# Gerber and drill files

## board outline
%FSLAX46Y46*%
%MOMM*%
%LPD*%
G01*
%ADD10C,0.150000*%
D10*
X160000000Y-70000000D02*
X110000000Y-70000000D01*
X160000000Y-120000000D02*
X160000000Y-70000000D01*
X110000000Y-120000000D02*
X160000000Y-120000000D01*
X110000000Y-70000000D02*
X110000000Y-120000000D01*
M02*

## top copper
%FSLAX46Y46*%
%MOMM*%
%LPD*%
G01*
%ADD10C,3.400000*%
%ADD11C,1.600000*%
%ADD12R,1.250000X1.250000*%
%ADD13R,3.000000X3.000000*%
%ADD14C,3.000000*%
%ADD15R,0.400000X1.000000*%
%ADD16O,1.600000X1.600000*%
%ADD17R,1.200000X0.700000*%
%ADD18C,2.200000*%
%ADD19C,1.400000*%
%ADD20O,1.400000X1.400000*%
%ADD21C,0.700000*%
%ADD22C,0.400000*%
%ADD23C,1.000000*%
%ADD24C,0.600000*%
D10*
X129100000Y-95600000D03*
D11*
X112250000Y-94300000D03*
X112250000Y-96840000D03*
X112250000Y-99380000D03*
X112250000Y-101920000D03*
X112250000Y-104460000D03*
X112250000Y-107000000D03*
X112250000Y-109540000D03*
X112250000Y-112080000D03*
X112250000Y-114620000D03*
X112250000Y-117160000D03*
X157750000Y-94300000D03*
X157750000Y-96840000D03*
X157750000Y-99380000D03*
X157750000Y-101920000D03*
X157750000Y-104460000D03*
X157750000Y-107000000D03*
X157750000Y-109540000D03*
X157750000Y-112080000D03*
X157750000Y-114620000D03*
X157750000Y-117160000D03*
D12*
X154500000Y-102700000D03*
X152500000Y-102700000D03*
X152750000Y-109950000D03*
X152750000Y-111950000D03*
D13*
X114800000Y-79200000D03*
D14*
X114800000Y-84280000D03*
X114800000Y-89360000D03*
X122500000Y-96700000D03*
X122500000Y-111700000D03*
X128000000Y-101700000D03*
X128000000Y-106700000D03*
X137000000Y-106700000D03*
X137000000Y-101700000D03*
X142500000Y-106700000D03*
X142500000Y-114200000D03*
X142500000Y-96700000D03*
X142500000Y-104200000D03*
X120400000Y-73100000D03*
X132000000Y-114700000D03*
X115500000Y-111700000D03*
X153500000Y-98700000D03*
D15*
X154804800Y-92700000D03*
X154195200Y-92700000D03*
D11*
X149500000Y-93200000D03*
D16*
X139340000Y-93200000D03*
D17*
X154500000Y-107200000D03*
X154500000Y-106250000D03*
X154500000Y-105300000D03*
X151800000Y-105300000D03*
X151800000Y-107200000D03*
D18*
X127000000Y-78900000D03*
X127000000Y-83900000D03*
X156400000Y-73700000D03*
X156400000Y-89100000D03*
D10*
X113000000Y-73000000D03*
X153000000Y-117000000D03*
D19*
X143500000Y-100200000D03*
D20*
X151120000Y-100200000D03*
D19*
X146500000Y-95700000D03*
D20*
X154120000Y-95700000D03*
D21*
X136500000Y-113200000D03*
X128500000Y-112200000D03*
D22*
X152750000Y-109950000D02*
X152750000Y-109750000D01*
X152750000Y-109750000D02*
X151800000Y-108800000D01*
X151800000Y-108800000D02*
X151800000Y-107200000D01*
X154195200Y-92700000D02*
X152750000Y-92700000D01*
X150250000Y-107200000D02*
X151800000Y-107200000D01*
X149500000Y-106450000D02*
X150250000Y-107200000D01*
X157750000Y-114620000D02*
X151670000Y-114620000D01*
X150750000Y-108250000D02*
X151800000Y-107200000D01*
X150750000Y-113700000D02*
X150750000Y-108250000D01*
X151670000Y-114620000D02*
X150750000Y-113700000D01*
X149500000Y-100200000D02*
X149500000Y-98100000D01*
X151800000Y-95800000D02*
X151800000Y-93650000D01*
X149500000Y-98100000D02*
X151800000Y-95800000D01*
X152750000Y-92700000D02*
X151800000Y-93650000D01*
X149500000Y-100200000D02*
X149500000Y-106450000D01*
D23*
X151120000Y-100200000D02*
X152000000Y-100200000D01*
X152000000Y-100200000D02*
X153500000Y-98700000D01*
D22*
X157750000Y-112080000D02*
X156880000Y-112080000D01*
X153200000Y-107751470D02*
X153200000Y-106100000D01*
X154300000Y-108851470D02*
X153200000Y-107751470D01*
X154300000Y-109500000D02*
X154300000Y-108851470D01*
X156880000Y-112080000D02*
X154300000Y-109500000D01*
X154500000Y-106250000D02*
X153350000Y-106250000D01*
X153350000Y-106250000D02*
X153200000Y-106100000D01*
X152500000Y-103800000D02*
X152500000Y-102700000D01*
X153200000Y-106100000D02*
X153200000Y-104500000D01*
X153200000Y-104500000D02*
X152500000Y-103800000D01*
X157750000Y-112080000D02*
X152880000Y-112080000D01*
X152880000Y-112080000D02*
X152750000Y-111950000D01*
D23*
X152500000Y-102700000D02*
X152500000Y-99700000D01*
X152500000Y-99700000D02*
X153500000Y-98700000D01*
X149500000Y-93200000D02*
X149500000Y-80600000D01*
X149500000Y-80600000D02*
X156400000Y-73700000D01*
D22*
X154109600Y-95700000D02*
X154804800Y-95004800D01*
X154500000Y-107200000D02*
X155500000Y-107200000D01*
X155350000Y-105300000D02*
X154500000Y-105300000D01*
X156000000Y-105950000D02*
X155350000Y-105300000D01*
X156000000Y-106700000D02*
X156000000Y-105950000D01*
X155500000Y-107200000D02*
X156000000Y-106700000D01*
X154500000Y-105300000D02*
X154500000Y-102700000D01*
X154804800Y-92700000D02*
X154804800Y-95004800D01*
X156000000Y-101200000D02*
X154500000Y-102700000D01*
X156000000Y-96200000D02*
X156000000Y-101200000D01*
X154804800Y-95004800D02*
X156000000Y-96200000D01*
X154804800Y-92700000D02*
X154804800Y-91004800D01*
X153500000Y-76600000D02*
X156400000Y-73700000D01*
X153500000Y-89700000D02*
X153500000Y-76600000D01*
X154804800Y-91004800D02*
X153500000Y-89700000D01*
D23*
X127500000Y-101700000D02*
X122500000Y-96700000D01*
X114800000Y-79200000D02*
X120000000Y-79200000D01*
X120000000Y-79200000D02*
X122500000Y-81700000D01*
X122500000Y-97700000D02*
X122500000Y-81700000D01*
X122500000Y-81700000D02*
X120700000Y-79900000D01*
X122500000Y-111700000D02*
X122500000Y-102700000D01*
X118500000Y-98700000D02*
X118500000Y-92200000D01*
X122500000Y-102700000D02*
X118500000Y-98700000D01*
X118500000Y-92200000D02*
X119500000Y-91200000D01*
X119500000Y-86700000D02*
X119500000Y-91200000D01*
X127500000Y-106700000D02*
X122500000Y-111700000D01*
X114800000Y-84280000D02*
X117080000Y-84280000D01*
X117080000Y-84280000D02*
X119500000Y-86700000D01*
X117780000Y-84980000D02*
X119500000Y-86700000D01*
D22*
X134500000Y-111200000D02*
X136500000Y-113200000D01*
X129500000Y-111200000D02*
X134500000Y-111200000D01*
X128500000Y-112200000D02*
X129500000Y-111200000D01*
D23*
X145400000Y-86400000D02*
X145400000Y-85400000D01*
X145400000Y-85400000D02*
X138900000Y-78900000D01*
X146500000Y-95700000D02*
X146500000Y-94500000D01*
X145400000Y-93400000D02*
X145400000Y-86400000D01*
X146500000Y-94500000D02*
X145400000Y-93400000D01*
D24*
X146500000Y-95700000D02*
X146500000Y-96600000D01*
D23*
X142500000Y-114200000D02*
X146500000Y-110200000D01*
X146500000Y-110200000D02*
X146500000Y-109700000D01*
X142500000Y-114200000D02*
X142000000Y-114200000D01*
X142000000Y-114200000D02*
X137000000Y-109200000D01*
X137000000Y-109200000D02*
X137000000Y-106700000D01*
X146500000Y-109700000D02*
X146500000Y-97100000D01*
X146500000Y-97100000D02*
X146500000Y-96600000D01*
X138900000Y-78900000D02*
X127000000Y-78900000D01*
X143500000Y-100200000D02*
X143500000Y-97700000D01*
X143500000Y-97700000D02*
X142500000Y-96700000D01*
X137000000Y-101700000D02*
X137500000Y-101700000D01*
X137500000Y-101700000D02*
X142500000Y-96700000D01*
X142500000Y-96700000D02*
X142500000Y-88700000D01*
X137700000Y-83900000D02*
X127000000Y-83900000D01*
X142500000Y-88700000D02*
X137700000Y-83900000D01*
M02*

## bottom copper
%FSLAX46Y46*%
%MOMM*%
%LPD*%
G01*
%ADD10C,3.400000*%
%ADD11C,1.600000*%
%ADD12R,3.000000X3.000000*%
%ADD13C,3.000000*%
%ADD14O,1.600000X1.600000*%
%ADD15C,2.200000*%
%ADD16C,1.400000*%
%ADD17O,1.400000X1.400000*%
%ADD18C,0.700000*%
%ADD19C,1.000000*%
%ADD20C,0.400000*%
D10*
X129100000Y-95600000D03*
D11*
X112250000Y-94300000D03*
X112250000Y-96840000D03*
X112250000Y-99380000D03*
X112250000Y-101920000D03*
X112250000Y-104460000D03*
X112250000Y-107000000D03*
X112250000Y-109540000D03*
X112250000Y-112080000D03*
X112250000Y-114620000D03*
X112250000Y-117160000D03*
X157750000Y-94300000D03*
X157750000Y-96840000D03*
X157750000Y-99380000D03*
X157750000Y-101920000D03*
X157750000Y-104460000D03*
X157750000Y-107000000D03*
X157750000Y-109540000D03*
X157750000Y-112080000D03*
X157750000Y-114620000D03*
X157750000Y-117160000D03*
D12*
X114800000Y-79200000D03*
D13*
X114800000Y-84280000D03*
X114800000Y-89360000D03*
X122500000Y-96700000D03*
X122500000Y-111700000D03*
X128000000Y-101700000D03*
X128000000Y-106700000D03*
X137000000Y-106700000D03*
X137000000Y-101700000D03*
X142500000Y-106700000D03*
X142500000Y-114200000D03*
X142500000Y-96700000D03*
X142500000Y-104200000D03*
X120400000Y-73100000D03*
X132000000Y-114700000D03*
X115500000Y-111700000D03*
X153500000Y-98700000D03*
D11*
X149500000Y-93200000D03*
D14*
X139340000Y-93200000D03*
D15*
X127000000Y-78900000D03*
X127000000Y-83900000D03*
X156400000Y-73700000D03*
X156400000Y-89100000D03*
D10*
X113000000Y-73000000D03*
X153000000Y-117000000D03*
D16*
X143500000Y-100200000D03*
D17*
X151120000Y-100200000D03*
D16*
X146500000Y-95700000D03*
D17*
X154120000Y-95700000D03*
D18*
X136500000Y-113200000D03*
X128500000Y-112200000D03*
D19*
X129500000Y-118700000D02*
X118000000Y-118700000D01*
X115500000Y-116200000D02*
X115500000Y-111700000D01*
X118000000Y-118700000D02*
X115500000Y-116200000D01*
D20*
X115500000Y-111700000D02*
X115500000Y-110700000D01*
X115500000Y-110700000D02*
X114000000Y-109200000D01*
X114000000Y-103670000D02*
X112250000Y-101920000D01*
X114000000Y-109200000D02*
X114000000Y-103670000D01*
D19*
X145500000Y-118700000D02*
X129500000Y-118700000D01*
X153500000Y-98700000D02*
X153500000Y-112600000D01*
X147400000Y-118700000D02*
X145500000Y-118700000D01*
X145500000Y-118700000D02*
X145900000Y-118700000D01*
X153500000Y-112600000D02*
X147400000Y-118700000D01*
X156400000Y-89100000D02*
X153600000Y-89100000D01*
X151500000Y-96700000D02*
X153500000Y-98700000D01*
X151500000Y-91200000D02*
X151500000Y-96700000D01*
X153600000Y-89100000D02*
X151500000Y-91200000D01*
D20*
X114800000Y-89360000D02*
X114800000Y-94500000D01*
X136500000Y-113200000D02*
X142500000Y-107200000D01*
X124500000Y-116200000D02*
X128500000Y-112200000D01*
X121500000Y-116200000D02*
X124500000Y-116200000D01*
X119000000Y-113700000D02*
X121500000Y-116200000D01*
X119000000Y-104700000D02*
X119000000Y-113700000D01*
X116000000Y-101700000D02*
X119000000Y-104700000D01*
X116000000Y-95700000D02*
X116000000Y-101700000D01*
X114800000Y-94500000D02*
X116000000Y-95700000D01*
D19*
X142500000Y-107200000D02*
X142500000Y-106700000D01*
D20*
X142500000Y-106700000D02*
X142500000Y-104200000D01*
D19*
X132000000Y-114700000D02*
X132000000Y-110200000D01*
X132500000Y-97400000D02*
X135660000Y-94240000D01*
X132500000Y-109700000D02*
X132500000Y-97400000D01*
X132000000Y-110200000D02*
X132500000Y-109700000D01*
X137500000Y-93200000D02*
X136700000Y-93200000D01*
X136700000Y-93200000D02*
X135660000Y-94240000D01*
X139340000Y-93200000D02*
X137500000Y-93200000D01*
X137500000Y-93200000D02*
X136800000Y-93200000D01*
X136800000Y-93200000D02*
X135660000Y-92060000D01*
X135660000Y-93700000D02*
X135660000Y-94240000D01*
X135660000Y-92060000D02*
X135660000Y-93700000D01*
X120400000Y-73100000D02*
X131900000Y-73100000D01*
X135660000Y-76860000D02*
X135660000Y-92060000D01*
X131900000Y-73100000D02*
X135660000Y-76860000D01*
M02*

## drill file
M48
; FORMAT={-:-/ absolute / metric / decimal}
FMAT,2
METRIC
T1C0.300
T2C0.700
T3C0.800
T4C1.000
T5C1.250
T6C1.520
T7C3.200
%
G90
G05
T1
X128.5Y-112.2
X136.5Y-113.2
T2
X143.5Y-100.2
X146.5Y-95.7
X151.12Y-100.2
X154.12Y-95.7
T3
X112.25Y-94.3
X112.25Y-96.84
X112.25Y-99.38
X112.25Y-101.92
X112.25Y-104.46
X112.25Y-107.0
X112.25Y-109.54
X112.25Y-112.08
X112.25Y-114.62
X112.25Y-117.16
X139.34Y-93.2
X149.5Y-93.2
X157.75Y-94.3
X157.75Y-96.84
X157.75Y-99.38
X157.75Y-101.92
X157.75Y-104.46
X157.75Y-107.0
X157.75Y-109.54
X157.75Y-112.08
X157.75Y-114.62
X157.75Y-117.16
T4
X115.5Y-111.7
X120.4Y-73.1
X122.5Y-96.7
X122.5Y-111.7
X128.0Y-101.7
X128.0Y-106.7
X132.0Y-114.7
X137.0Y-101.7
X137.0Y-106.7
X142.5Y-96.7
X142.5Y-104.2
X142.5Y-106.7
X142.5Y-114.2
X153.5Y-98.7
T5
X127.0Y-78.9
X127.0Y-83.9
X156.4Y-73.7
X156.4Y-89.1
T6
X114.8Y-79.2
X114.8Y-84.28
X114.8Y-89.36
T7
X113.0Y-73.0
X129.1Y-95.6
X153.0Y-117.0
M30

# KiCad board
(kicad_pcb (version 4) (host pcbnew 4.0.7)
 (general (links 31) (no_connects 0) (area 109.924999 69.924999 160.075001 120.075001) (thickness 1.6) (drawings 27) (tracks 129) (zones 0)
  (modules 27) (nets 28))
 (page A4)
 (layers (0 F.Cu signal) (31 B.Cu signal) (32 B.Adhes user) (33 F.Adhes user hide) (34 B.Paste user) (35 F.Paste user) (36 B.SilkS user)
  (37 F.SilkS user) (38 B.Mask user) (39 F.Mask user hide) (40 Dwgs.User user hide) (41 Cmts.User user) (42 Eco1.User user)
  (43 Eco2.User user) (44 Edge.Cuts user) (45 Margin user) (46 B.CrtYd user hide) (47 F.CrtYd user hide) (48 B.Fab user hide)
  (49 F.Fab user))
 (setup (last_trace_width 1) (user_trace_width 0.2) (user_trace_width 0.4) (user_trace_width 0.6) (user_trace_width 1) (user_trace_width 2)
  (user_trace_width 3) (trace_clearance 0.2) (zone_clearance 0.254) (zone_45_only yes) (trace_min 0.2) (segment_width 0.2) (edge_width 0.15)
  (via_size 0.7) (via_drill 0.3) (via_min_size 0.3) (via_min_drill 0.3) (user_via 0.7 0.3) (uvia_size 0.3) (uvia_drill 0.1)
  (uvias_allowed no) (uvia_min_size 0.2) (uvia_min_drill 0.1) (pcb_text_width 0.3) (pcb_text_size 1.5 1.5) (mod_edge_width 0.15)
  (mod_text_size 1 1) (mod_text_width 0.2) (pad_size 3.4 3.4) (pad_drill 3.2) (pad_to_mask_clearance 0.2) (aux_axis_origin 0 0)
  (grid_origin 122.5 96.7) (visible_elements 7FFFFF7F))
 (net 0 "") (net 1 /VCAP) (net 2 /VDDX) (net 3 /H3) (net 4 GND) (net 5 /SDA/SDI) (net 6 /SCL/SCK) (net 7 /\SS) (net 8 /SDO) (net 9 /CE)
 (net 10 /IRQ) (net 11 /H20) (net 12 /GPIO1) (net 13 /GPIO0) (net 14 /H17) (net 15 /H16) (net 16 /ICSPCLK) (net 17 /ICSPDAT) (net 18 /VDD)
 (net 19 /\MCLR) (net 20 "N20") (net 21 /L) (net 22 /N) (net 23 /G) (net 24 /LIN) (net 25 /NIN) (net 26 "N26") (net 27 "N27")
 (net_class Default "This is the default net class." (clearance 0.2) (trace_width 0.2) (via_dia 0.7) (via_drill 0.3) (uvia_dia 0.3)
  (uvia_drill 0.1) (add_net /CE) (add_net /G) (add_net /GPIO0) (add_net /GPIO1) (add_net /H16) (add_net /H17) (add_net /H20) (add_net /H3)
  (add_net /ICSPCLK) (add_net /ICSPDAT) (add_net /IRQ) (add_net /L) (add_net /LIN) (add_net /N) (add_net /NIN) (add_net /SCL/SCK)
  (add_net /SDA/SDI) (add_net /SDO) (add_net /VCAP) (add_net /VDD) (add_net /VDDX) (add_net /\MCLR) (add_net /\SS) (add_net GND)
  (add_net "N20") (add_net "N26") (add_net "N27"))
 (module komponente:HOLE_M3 (layer F.Cu) (at 129.1 95.6)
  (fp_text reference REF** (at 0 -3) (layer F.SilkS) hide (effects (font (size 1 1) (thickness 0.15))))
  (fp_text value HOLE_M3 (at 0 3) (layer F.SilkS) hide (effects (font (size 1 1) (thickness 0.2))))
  (pad 1 thru_hole circle (at 0 0) (size 3.4 3.4) (drill 3.2) (layers *.Cu *.Mask F.SilkS)))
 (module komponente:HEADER (layer F.Cu) (at 135 107)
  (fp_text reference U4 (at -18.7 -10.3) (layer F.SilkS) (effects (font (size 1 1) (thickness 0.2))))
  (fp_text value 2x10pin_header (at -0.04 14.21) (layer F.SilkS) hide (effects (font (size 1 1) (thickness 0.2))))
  (pad 1 thru_hole circle (at -22.75 -12.7) (size 1.6 1.6) (drill 0.8) (layers *.Cu *.Mask F.SilkS) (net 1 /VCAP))
  (pad 2 thru_hole circle (at -22.75 -10.16) (size 1.6 1.6) (drill 0.8) (layers *.Cu *.Mask F.SilkS) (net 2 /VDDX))
  (pad 3 thru_hole circle (at -22.75 -7.62) (size 1.6 1.6) (drill 0.8) (layers *.Cu *.Mask F.SilkS) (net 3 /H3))
  (pad 4 thru_hole circle (at -22.75 -5.08) (size 1.6 1.6) (drill 0.8) (layers *.Cu *.Mask F.SilkS) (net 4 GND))
  (pad 5 thru_hole circle (at -22.75 -2.54) (size 1.6 1.6) (drill 0.8) (layers *.Cu *.Mask F.SilkS) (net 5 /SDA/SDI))
  (pad 6 thru_hole circle (at -22.75 0) (size 1.6 1.6) (drill 0.8) (layers *.Cu *.Mask F.SilkS) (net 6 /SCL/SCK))
  (pad 7 thru_hole circle (at -22.75 2.54) (size 1.6 1.6) (drill 0.8) (layers *.Cu *.Mask F.SilkS) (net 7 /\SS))
  (pad 8 thru_hole circle (at -22.75 5.08) (size 1.6 1.6) (drill 0.8) (layers *.Cu *.Mask F.SilkS) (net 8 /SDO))
  (pad 9 thru_hole circle (at -22.75 7.62) (size 1.6 1.6) (drill 0.8) (layers *.Cu *.Mask F.SilkS) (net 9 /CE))
  (pad 10 thru_hole circle (at -22.75 10.16) (size 1.6 1.6) (drill 0.8) (layers *.Cu *.Mask F.SilkS) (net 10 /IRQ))
  (pad 20 thru_hole circle (at 22.75 -12.7) (size 1.6 1.6) (drill 0.8) (layers *.Cu *.Mask F.SilkS) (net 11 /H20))
  (pad 19 thru_hole circle (at 22.75 -10.16) (size 1.6 1.6) (drill 0.8) (layers *.Cu *.Mask F.SilkS) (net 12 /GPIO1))
  (pad 18 thru_hole circle (at 22.75 -7.62) (size 1.6 1.6) (drill 0.8) (layers *.Cu *.Mask F.SilkS) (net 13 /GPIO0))
  (pad 17 thru_hole circle (at 22.75 -5.08) (size 1.6 1.6) (drill 0.8) (layers *.Cu *.Mask F.SilkS) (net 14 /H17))
  (pad 16 thru_hole circle (at 22.75 -2.54) (size 1.6 1.6) (drill 0.8) (layers *.Cu *.Mask F.SilkS) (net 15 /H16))
  (pad 15 thru_hole circle (at 22.75 0) (size 1.6 1.6) (drill 0.8) (layers *.Cu *.Mask F.SilkS) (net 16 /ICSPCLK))
  (pad 14 thru_hole circle (at 22.75 2.54) (size 1.6 1.6) (drill 0.8) (layers *.Cu *.Mask F.SilkS) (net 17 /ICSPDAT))
  (pad 13 thru_hole circle (at 22.75 5.08) (size 1.6 1.6) (drill 0.8) (layers *.Cu *.Mask F.SilkS) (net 4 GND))
  (pad 12 thru_hole circle (at 22.75 7.62) (size 1.6 1.6) (drill 0.8) (layers *.Cu *.Mask F.SilkS) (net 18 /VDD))
  (pad 11 thru_hole circle (at 22.75 10.16) (size 1.6 1.6) (drill 0.8) (layers *.Cu *.Mask F.SilkS) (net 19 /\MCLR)))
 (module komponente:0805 (layer F.Cu) (at 153.5 102.7 180)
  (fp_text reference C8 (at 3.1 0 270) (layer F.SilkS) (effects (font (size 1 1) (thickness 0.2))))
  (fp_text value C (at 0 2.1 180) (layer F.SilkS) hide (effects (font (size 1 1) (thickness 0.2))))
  (pad 1 smd rect (at -1 0 180) (size 1.25 1.25) (layers F.Cu F.Paste F.Mask) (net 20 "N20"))
  (pad 2 smd rect (at 1 0 180) (size 1.25 1.25) (layers F.Cu F.Paste F.Mask) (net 4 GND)))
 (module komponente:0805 (layer F.Cu) (at 152.75 110.95 270)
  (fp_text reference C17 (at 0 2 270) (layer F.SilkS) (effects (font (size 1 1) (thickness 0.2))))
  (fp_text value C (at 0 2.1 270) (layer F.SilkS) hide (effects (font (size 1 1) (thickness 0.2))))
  (pad 1 smd rect (at -1 0 270) (size 1.25 1.25) (layers F.Cu F.Paste F.Mask) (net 18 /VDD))
  (pad 2 smd rect (at 1 0 270) (size 1.25 1.25) (layers F.Cu F.Paste F.Mask) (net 4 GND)))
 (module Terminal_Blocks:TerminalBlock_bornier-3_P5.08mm (layer F.Cu) (at 114.8 79.2 270)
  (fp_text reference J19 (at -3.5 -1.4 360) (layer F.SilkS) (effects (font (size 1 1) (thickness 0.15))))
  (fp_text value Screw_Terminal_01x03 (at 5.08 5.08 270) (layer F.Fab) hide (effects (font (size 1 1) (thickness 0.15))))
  (pad 1 thru_hole rect (at 0 0 270) (size 3 3) (drill 1.52) (layers *.Cu *.Mask) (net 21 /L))
  (pad 2 thru_hole circle (at 5.08 0 270) (size 3 3) (drill 1.52) (layers *.Cu *.Mask) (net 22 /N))
  (pad 3 thru_hole circle (at 10.16 0 270) (size 3 3) (drill 1.52) (layers *.Cu *.Mask) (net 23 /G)))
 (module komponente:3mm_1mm (layer F.Cu) (at 122.5 96.7)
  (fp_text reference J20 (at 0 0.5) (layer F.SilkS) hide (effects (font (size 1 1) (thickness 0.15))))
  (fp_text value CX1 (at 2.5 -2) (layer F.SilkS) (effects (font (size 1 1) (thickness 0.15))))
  (pad 1 thru_hole circle (at 0 0) (size 3 3) (drill 1) (layers *.Cu *.Mask) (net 21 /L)))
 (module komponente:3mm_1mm (layer F.Cu) (at 122.5 111.7)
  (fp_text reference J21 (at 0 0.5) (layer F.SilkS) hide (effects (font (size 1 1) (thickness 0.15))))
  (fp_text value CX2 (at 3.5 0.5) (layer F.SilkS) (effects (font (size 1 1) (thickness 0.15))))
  (pad 1 thru_hole circle (at 0 0) (size 3 3) (drill 1) (layers *.Cu *.Mask) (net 22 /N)))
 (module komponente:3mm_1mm (layer F.Cu) (at 128 101.7)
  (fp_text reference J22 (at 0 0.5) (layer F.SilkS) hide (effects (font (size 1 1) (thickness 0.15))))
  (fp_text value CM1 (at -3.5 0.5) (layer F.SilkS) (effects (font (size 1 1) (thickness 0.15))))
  (pad 1 thru_hole circle (at 0 0) (size 3 3) (drill 1) (layers *.Cu *.Mask) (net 21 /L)))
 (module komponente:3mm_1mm (layer F.Cu) (at 128 106.7)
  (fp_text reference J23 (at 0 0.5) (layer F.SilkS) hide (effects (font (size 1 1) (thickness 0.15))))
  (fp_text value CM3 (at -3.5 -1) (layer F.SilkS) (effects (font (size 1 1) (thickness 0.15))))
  (pad 1 thru_hole circle (at 0 0) (size 3 3) (drill 1) (layers *.Cu *.Mask) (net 22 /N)))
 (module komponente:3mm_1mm (layer F.Cu) (at 137 106.7)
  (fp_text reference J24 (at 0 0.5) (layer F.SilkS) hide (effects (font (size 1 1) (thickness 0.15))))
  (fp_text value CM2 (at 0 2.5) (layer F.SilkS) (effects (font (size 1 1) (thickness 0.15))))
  (pad 1 thru_hole circle (at 0 0) (size 3 3) (drill 1) (layers *.Cu *.Mask) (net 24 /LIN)))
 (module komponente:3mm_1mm (layer F.Cu) (at 137 101.7)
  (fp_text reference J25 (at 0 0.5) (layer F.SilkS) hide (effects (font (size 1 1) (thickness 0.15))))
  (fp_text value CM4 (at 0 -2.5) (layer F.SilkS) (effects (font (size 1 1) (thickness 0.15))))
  (pad 1 thru_hole circle (at 0 0) (size 3 3) (drill 1) (layers *.Cu *.Mask) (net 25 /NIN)))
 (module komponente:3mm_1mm (layer F.Cu) (at 142.5 106.7)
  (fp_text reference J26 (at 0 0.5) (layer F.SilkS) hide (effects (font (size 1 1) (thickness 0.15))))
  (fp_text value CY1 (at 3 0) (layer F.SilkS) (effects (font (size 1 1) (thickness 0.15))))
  (pad 1 thru_hole circle (at 0 0) (size 3 3) (drill 1) (layers *.Cu *.Mask) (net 23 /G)))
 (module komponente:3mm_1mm (layer F.Cu) (at 142.5 114.2)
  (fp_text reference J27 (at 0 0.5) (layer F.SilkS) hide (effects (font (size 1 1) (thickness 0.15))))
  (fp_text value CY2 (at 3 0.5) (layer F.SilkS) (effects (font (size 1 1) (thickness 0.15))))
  (pad 1 thru_hole circle (at 0 0) (size 3 3) (drill 1) (layers *.Cu *.Mask) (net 24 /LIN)))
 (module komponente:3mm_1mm (layer F.Cu) (at 142.5 96.7)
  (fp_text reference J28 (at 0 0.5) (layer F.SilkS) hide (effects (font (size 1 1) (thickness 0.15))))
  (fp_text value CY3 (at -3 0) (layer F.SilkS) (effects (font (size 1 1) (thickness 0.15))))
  (pad 1 thru_hole circle (at 0 0) (size 3 3) (drill 1) (layers *.Cu *.Mask) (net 25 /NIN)))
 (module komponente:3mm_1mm (layer F.Cu) (at 142.5 104.2)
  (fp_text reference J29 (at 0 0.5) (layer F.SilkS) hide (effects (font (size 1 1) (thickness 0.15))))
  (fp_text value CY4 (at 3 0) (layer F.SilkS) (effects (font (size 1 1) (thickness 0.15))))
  (pad 1 thru_hole circle (at 0 0) (size 3 3) (drill 1) (layers *.Cu *.Mask) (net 23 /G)))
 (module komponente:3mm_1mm (layer F.Cu) (at 120.4 73.1)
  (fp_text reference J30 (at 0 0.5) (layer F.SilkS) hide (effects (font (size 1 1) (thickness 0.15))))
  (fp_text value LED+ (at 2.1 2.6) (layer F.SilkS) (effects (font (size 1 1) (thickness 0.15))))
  (pad 1 thru_hole circle (at 0 0) (size 3 3) (drill 1) (layers *.Cu *.Mask) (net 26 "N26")))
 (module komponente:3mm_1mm (layer F.Cu) (at 132 114.7)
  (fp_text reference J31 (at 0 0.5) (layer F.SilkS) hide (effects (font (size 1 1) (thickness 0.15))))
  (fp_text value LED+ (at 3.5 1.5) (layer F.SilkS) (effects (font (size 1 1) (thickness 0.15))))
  (pad 1 thru_hole circle (at 0 0) (size 3 3) (drill 1) (layers *.Cu *.Mask) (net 26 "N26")))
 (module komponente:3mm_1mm (layer F.Cu) (at 115.5 111.7)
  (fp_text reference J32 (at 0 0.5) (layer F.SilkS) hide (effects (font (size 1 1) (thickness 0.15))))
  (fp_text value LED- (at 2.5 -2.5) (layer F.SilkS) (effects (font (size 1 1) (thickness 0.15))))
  (pad 1 thru_hole circle (at 0 0) (size 3 3) (drill 1) (layers *.Cu *.Mask) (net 4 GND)))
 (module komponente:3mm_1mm (layer F.Cu) (at 153.5 98.7)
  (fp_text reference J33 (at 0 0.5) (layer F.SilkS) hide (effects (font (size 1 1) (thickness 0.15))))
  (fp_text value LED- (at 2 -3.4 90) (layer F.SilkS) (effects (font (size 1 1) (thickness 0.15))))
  (pad 1 thru_hole circle (at 0 0) (size 3 3) (drill 1) (layers *.Cu *.Mask) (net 4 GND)))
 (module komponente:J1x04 (layer F.Cu) (at 154.5 92.7 180)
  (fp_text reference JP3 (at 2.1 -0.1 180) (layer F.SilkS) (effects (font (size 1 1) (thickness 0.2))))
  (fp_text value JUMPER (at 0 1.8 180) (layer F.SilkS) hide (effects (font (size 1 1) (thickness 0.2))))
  (pad 1 smd rect (at -0.3048 0 180) (size 0.4 1) (layers F.Cu F.Paste F.Mask) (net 20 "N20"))
  (pad 2 smd rect (at 0.3048 0 180) (size 0.4 1) (layers F.Cu F.Paste F.Mask) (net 18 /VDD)))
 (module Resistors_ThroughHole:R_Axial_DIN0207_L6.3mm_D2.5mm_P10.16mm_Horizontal (layer F.Cu) (at 149.5 93.2 180)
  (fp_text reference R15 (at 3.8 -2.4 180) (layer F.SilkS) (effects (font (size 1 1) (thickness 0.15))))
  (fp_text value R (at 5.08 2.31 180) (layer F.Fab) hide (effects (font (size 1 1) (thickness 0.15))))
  (pad 1 thru_hole circle (at 0 0 180) (size 1.6 1.6) (drill 0.8) (layers *.Cu *.Mask) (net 20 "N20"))
  (pad 2 thru_hole oval (at 10.16 0 180) (size 1.6 1.6) (drill 0.8) (layers *.Cu *.Mask) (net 26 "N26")))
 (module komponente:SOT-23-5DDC (layer F.Cu) (at 154.5 107.2 90)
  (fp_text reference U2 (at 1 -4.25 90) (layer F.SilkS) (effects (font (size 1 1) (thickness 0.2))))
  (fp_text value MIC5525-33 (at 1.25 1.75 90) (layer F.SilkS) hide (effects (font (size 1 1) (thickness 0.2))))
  (pad 1 smd rect (at 0 0 90) (size 0.7 1.2) (layers F.Cu F.Paste F.Mask) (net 20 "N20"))
  (pad 2 smd rect (at 0.95 0 90) (size 0.7 1.2) (layers F.Cu F.Paste F.Mask) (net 4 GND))
  (pad 3 smd rect (at 1.9 0 90) (size 0.7 1.2) (layers F.Cu F.Paste F.Mask) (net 20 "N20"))
  (pad 4 smd rect (at 1.9 -2.7 90) (size 0.7 1.2) (layers F.Cu F.Paste F.Mask) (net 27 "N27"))
  (pad 5 smd rect (at 0 -2.7 90) (size 0.7 1.2) (layers F.Cu F.Paste F.Mask) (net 18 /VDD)))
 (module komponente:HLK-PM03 (layer F.Cu) (at 141.7 81.4)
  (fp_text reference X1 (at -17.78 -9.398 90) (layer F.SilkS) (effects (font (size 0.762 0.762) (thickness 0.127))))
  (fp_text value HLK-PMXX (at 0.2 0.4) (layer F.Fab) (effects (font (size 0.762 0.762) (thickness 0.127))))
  (pad 1 thru_hole circle (at -14.7 -2.5) (size 2.2 2.2) (drill 1.25) (layers *.Cu *.Mask) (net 24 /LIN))
  (pad 2 thru_hole circle (at -14.7 2.5) (size 2.2 2.2) (drill 1.25) (layers *.Cu *.Mask) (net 25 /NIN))
  (pad 3 thru_hole circle (at 14.7 -7.7) (size 2.2 2.2) (drill 1.25) (layers *.Cu *.Mask) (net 20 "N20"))
  (pad 4 thru_hole circle (at 14.7 7.7) (size 2.2 2.2) (drill 1.25) (layers *.Cu *.Mask) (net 4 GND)))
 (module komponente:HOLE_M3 (layer F.Cu) (at 113 73)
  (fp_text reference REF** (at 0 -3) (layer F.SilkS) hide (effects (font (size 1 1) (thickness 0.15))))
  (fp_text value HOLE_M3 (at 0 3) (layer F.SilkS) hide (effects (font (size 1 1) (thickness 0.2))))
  (pad 1 thru_hole circle (at 0 0) (size 3.4 3.4) (drill 3.2) (layers *.Cu *.Mask F.SilkS)))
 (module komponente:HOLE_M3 (layer F.Cu) (at 153 117)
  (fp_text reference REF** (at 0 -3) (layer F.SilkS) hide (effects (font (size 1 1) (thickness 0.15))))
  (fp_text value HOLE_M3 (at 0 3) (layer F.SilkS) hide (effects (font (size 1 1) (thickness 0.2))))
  (pad 1 thru_hole circle (at 0 0) (size 3.4 3.4) (drill 3.2) (layers *.Cu *.Mask F.SilkS)))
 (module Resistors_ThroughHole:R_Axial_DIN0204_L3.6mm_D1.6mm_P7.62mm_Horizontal (layer F.Cu) (at 143.5 100.2)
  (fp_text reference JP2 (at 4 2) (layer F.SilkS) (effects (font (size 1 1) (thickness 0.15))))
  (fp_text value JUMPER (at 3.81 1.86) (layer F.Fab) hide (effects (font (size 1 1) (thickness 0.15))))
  (pad 1 thru_hole circle (at 0 0) (size 1.4 1.4) (drill 0.7) (layers *.Cu *.Mask) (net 25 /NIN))
  (pad 2 thru_hole oval (at 7.62 0) (size 1.4 1.4) (drill 0.7) (layers *.Cu *.Mask) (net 4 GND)))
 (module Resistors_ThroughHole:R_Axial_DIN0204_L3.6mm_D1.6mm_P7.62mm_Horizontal (layer F.Cu) (at 146.5 95.7)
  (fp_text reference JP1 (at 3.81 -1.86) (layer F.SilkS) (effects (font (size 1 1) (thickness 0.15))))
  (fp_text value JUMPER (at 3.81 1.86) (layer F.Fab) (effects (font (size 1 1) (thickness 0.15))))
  (pad 1 thru_hole circle (at 0 0) (size 1.4 1.4) (drill 0.7) (layers *.Cu *.Mask) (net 24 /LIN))
  (pad 2 thru_hole oval (at 7.62 0) (size 1.4 1.4) (drill 0.7) (layers *.Cu *.Mask) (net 20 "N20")))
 (gr_line (start 160 70) (end 110 70) (angle 90) (layer Edge.Cuts) (width 0.15))
 (gr_line (start 160 120) (end 160 70) (angle 90) (layer Edge.Cuts) (width 0.15))
 (gr_line (start 110 120) (end 160 120) (angle 90) (layer Edge.Cuts) (width 0.15))
 (gr_line (start 110 70) (end 110 120) (angle 90) (layer Edge.Cuts) (width 0.15))
 (segment (start 152.75 109.95) (end 152.75 109.75) (width 0.4) (layer F.Cu) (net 18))
 (segment (start 152.75 109.75) (end 151.8 108.8) (width 0.4) (layer F.Cu) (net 18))
 (segment (start 151.8 108.8) (end 151.8 107.2) (width 0.4) (layer F.Cu) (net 18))
 (segment (start 154.1952 92.7) (end 152.75 92.7) (width 0.4) (layer F.Cu) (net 18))
 (segment (start 150.25 107.2) (end 151.8 107.2) (width 0.4) (layer F.Cu) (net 18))
 (segment (start 149.5 106.45) (end 150.25 107.2) (width 0.4) (layer F.Cu) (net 18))
 (segment (start 157.75 114.62) (end 151.67 114.62) (width 0.4) (layer F.Cu) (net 18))
 (segment (start 150.75 108.25) (end 151.8 107.2) (width 0.4) (layer F.Cu) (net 18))
 (segment (start 150.75 113.7) (end 150.75 108.25) (width 0.4) (layer F.Cu) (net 18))
 (segment (start 151.67 114.62) (end 150.75 113.7) (width 0.4) (layer F.Cu) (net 18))
 (segment (start 149.5 100.2) (end 149.5 98.1) (width 0.4) (layer F.Cu) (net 18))
 (segment (start 151.8 95.8) (end 151.8 93.65) (width 0.4) (layer F.Cu) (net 18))
 (segment (start 149.5 98.1) (end 151.8 95.8) (width 0.4) (layer F.Cu) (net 18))
 (segment (start 152.75 92.7) (end 151.8 93.65) (width 0.4) (layer F.Cu) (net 18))
 (segment (start 149.5 100.2) (end 149.5 106.45) (width 0.4) (layer F.Cu) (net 18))
 (segment (start 129.5 118.7) (end 118 118.7) (width 1) (layer B.Cu) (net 4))
 (segment (start 115.5 116.2) (end 115.5 111.7) (width 1) (layer B.Cu) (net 4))
 (segment (start 118 118.7) (end 115.5 116.2) (width 1) (layer B.Cu) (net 4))
 (segment (start 115.5 111.7) (end 115.5 110.7) (width 0.4) (layer B.Cu) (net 4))
 (segment (start 115.5 110.7) (end 114 109.2) (width 0.4) (layer B.Cu) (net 4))
 (segment (start 114 103.67) (end 112.25 101.92) (width 0.4) (layer B.Cu) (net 4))
 (segment (start 114 109.2) (end 114 103.67) (width 0.4) (layer B.Cu) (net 4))
 (segment (start 151.12 100.2) (end 152 100.2) (width 1) (layer F.Cu) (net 4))
 (segment (start 152 100.2) (end 153.5 98.7) (width 1) (layer F.Cu) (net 4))
 (segment (start 145.5 118.7) (end 129.5 118.7) (width 1) (layer B.Cu) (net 4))
 (segment (start 153.5 98.7) (end 153.5 112.6) (width 1) (layer B.Cu) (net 4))
 (segment (start 147.4 118.7) (end 145.5 118.7) (width 1) (layer B.Cu) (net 4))
 (segment (start 145.5 118.7) (end 145.9 118.7) (width 1) (layer B.Cu) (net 4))
 (segment (start 153.5 112.6) (end 147.4 118.7) (width 1) (layer B.Cu) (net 4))
 (segment (start 157.75 112.08) (end 156.88 112.08) (width 0.4) (layer F.Cu) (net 4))
 (segment (start 153.2 107.75147) (end 153.2 106.1) (width 0.4) (layer F.Cu) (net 4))
 (segment (start 154.3 108.85147) (end 153.2 107.75147) (width 0.4) (layer F.Cu) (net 4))
 (segment (start 154.3 109.5) (end 154.3 108.85147) (width 0.4) (layer F.Cu) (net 4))
 (segment (start 156.88 112.08) (end 154.3 109.5) (width 0.4) (layer F.Cu) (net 4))
 (segment (start 154.5 106.25) (end 153.35 106.25) (width 0.4) (layer F.Cu) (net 4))
 (segment (start 153.35 106.25) (end 153.2 106.1) (width 0.4) (layer F.Cu) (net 4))
 (segment (start 152.5 103.8) (end 152.5 102.7) (width 0.4) (layer F.Cu) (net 4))
 (segment (start 153.2 106.1) (end 153.2 104.5) (width 0.4) (layer F.Cu) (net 4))
 (segment (start 153.2 104.5) (end 152.5 103.8) (width 0.4) (layer F.Cu) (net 4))
 (segment (start 157.75 112.08) (end 152.88 112.08) (width 0.4) (layer F.Cu) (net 4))
 (segment (start 152.88 112.08) (end 152.75 111.95) (width 0.4) (layer F.Cu) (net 4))
 (segment (start 152.5 102.7) (end 152.5 99.7) (width 1) (layer F.Cu) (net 4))
 (segment (start 152.5 99.7) (end 153.5 98.7) (width 1) (layer F.Cu) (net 4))
 (segment (start 156.4 89.1) (end 153.6 89.1) (width 1) (layer B.Cu) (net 4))
 (segment (start 151.5 96.7) (end 153.5 98.7) (width 1) (layer B.Cu) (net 4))
 (segment (start 151.5 91.2) (end 151.5 96.7) (width 1) (layer B.Cu) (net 4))
 (segment (start 153.6 89.1) (end 151.5 91.2) (width 1) (layer B.Cu) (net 4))
 (segment (start 149.5 93.2) (end 149.5 80.6) (width 1) (layer F.Cu) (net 20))
 (segment (start 149.5 80.6) (end 156.4 73.7) (width 1) (layer F.Cu) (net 20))
 (segment (start 154.1096 95.7) (end 154.8048 95.0048) (width 0.4) (layer F.Cu) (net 20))
 (segment (start 154.5 107.2) (end 155.5 107.2) (width 0.4) (layer F.Cu) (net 20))
 (segment (start 155.35 105.3) (end 154.5 105.3) (width 0.4) (layer F.Cu) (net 20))
 (segment (start 156 105.95) (end 155.35 105.3) (width 0.4) (layer F.Cu) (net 20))
 (segment (start 156 106.7) (end 156 105.95) (width 0.4) (layer F.Cu) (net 20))
 (segment (start 155.5 107.2) (end 156 106.7) (width 0.4) (layer F.Cu) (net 20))
 (segment (start 154.5 105.3) (end 154.5 102.7) (width 0.4) (layer F.Cu) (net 20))
 (segment (start 154.8048 92.7) (end 154.8048 95.0048) (width 0.4) (layer F.Cu) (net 20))
 (segment (start 156 101.2) (end 154.5 102.7) (width 0.4) (layer F.Cu) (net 20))
 (segment (start 156 96.2) (end 156 101.2) (width 0.4) (layer F.Cu) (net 20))
 (segment (start 154.8048 95.0048) (end 156 96.2) (width 0.4) (layer F.Cu) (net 20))
 (segment (start 154.8048 92.7) (end 154.8048 91.0048) (width 0.4) (layer F.Cu) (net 20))
 (segment (start 153.5 76.6) (end 156.4 73.7) (width 0.4) (layer F.Cu) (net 20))
 (segment (start 153.5 89.7) (end 153.5 76.6) (width 0.4) (layer F.Cu) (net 20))
 (segment (start 154.8048 91.0048) (end 153.5 89.7) (width 0.4) (layer F.Cu) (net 20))
 (segment (start 127.5 101.7) (end 122.5 96.7) (width 1) (layer F.Cu) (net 21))
 (segment (start 114.8 79.2) (end 120 79.2) (width 1) (layer F.Cu) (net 21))
 (segment (start 120 79.2) (end 122.5 81.7) (width 1) (layer F.Cu) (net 21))
 (segment (start 122.5 97.7) (end 122.5 81.7) (width 1) (layer F.Cu) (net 21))
 (segment (start 122.5 81.7) (end 120.7 79.9) (width 1) (layer F.Cu) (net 21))
 (segment (start 122.5 111.7) (end 122.5 102.7) (width 1) (layer F.Cu) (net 22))
 (segment (start 118.5 98.7) (end 118.5 92.2) (width 1) (layer F.Cu) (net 22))
 (segment (start 122.5 102.7) (end 118.5 98.7) (width 1) (layer F.Cu) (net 22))
 (segment (start 118.5 92.2) (end 119.5 91.2) (width 1) (layer F.Cu) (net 22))
 (segment (start 119.5 86.7) (end 119.5 91.2) (width 1) (layer F.Cu) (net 22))
 (segment (start 127.5 106.7) (end 122.5 111.7) (width 1) (layer F.Cu) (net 22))
 (segment (start 114.8 84.28) (end 117.08 84.28) (width 1) (layer F.Cu) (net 22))
 (segment (start 117.08 84.28) (end 119.5 86.7) (width 1) (layer F.Cu) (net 22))
 (segment (start 117.78 84.98) (end 119.5 86.7) (width 1) (layer F.Cu) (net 22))
 (segment (start 114.8 89.36) (end 114.8 94.5) (width 0.4) (layer B.Cu) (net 23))
 (segment (start 136.5 113.2) (end 142.5 107.2) (width 0.4) (layer B.Cu) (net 23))
 (via (at 136.5 113.2) (size 0.7) (drill 0.3) (layers F.Cu B.Cu) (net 23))
 (segment (start 134.5 111.2) (end 136.5 113.2) (width 0.4) (layer F.Cu) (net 23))
 (segment (start 129.5 111.2) (end 134.5 111.2) (width 0.4) (layer F.Cu) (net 23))
 (segment (start 128.5 112.2) (end 129.5 111.2) (width 0.4) (layer F.Cu) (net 23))
 (via (at 128.5 112.2) (size 0.7) (drill 0.3) (layers F.Cu B.Cu) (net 23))
 (segment (start 124.5 116.2) (end 128.5 112.2) (width 0.4) (layer B.Cu) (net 23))
 (segment (start 121.5 116.2) (end 124.5 116.2) (width 0.4) (layer B.Cu) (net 23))
 (segment (start 119 113.7) (end 121.5 116.2) (width 0.4) (layer B.Cu) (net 23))
 (segment (start 119 104.7) (end 119 113.7) (width 0.4) (layer B.Cu) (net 23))
 (segment (start 116 101.7) (end 119 104.7) (width 0.4) (layer B.Cu) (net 23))
 (segment (start 116 95.7) (end 116 101.7) (width 0.4) (layer B.Cu) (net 23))
 (segment (start 114.8 94.5) (end 116 95.7) (width 0.4) (layer B.Cu) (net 23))
 (segment (start 142.5 107.2) (end 142.5 106.7) (width 1) (layer B.Cu) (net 23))
 (segment (start 142.5 106.7) (end 142.5 104.2) (width 0.4) (layer B.Cu) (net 23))
 (segment (start 145.4 86.4) (end 145.4 85.4) (width 1) (layer F.Cu) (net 24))
 (segment (start 145.4 85.4) (end 138.9 78.9) (width 1) (layer F.Cu) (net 24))
 (segment (start 146.5 95.7) (end 146.5 94.5) (width 1) (layer F.Cu) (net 24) (status 400000))
 (segment (start 145.4 93.4) (end 145.4 86.4) (width 1) (layer F.Cu) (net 24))
 (segment (start 146.5 94.5) (end 145.4 93.4) (width 1) (layer F.Cu) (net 24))
 (segment (start 146.5 95.7) (end 146.5 96.6) (width 0.6) (layer F.Cu) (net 24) (status 400000))
 (segment (start 142.5 114.2) (end 146.5 110.2) (width 1) (layer F.Cu) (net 24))
 (segment (start 146.5 110.2) (end 146.5 109.7) (width 1) (layer F.Cu) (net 24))
 (segment (start 142.5 114.2) (end 142 114.2) (width 1) (layer F.Cu) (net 24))
 (segment (start 142 114.2) (end 137 109.2) (width 1) (layer F.Cu) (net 24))
 (segment (start 137 109.2) (end 137 106.7) (width 1) (layer F.Cu) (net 24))
 (segment (start 146.5 109.7) (end 146.5 97.1) (width 1) (layer F.Cu) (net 24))
 (segment (start 146.5 97.1) (end 146.5 96.6) (width 1) (layer F.Cu) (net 24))
 (segment (start 138.9 78.9) (end 127 78.9) (width 1) (layer F.Cu) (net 24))
 (segment (start 143.5 100.2) (end 143.5 97.7) (width 1) (layer F.Cu) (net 25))
 (segment (start 143.5 97.7) (end 142.5 96.7) (width 1) (layer F.Cu) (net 25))
 (segment (start 137 101.7) (end 137.5 101.7) (width 1) (layer F.Cu) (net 25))
 (segment (start 137.5 101.7) (end 142.5 96.7) (width 1) (layer F.Cu) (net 25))
 (segment (start 142.5 96.7) (end 142.5 88.7) (width 1) (layer F.Cu) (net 25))
 (segment (start 137.7 83.9) (end 127 83.9) (width 1) (layer F.Cu) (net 25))
 (segment (start 142.5 88.7) (end 137.7 83.9) (width 1) (layer F.Cu) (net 25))
 (segment (start 132 114.7) (end 132 110.2) (width 1) (layer B.Cu) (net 26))
 (segment (start 132.5 97.4) (end 135.66 94.24) (width 1) (layer B.Cu) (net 26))
 (segment (start 132.5 109.7) (end 132.5 97.4) (width 1) (layer B.Cu) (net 26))
 (segment (start 132 110.2) (end 132.5 109.7) (width 1) (layer B.Cu) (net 26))
 (segment (start 137.5 93.2) (end 136.7 93.2) (width 1) (layer B.Cu) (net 26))
 (segment (start 136.7 93.2) (end 135.66 94.24) (width 1) (layer B.Cu) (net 26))
 (segment (start 139.34 93.2) (end 137.5 93.2) (width 1) (layer B.Cu) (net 26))
 (segment (start 137.5 93.2) (end 136.8 93.2) (width 1) (layer B.Cu) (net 26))
 (segment (start 136.8 93.2) (end 135.66 92.06) (width 1) (layer B.Cu) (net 26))
 (segment (start 135.66 93.7) (end 135.66 94.24) (width 1) (layer B.Cu) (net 26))
 (segment (start 135.66 92.06) (end 135.66 93.7) (width 1) (layer B.Cu) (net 26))
 (segment (start 120.4 73.1) (end 131.9 73.1) (width 1) (layer B.Cu) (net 26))
 (segment (start 135.66 76.86) (end 135.66 92.06) (width 1) (layer B.Cu) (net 26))
 (segment (start 131.9 73.1) (end 135.66 76.86) (width 1) (layer B.Cu) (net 26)))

